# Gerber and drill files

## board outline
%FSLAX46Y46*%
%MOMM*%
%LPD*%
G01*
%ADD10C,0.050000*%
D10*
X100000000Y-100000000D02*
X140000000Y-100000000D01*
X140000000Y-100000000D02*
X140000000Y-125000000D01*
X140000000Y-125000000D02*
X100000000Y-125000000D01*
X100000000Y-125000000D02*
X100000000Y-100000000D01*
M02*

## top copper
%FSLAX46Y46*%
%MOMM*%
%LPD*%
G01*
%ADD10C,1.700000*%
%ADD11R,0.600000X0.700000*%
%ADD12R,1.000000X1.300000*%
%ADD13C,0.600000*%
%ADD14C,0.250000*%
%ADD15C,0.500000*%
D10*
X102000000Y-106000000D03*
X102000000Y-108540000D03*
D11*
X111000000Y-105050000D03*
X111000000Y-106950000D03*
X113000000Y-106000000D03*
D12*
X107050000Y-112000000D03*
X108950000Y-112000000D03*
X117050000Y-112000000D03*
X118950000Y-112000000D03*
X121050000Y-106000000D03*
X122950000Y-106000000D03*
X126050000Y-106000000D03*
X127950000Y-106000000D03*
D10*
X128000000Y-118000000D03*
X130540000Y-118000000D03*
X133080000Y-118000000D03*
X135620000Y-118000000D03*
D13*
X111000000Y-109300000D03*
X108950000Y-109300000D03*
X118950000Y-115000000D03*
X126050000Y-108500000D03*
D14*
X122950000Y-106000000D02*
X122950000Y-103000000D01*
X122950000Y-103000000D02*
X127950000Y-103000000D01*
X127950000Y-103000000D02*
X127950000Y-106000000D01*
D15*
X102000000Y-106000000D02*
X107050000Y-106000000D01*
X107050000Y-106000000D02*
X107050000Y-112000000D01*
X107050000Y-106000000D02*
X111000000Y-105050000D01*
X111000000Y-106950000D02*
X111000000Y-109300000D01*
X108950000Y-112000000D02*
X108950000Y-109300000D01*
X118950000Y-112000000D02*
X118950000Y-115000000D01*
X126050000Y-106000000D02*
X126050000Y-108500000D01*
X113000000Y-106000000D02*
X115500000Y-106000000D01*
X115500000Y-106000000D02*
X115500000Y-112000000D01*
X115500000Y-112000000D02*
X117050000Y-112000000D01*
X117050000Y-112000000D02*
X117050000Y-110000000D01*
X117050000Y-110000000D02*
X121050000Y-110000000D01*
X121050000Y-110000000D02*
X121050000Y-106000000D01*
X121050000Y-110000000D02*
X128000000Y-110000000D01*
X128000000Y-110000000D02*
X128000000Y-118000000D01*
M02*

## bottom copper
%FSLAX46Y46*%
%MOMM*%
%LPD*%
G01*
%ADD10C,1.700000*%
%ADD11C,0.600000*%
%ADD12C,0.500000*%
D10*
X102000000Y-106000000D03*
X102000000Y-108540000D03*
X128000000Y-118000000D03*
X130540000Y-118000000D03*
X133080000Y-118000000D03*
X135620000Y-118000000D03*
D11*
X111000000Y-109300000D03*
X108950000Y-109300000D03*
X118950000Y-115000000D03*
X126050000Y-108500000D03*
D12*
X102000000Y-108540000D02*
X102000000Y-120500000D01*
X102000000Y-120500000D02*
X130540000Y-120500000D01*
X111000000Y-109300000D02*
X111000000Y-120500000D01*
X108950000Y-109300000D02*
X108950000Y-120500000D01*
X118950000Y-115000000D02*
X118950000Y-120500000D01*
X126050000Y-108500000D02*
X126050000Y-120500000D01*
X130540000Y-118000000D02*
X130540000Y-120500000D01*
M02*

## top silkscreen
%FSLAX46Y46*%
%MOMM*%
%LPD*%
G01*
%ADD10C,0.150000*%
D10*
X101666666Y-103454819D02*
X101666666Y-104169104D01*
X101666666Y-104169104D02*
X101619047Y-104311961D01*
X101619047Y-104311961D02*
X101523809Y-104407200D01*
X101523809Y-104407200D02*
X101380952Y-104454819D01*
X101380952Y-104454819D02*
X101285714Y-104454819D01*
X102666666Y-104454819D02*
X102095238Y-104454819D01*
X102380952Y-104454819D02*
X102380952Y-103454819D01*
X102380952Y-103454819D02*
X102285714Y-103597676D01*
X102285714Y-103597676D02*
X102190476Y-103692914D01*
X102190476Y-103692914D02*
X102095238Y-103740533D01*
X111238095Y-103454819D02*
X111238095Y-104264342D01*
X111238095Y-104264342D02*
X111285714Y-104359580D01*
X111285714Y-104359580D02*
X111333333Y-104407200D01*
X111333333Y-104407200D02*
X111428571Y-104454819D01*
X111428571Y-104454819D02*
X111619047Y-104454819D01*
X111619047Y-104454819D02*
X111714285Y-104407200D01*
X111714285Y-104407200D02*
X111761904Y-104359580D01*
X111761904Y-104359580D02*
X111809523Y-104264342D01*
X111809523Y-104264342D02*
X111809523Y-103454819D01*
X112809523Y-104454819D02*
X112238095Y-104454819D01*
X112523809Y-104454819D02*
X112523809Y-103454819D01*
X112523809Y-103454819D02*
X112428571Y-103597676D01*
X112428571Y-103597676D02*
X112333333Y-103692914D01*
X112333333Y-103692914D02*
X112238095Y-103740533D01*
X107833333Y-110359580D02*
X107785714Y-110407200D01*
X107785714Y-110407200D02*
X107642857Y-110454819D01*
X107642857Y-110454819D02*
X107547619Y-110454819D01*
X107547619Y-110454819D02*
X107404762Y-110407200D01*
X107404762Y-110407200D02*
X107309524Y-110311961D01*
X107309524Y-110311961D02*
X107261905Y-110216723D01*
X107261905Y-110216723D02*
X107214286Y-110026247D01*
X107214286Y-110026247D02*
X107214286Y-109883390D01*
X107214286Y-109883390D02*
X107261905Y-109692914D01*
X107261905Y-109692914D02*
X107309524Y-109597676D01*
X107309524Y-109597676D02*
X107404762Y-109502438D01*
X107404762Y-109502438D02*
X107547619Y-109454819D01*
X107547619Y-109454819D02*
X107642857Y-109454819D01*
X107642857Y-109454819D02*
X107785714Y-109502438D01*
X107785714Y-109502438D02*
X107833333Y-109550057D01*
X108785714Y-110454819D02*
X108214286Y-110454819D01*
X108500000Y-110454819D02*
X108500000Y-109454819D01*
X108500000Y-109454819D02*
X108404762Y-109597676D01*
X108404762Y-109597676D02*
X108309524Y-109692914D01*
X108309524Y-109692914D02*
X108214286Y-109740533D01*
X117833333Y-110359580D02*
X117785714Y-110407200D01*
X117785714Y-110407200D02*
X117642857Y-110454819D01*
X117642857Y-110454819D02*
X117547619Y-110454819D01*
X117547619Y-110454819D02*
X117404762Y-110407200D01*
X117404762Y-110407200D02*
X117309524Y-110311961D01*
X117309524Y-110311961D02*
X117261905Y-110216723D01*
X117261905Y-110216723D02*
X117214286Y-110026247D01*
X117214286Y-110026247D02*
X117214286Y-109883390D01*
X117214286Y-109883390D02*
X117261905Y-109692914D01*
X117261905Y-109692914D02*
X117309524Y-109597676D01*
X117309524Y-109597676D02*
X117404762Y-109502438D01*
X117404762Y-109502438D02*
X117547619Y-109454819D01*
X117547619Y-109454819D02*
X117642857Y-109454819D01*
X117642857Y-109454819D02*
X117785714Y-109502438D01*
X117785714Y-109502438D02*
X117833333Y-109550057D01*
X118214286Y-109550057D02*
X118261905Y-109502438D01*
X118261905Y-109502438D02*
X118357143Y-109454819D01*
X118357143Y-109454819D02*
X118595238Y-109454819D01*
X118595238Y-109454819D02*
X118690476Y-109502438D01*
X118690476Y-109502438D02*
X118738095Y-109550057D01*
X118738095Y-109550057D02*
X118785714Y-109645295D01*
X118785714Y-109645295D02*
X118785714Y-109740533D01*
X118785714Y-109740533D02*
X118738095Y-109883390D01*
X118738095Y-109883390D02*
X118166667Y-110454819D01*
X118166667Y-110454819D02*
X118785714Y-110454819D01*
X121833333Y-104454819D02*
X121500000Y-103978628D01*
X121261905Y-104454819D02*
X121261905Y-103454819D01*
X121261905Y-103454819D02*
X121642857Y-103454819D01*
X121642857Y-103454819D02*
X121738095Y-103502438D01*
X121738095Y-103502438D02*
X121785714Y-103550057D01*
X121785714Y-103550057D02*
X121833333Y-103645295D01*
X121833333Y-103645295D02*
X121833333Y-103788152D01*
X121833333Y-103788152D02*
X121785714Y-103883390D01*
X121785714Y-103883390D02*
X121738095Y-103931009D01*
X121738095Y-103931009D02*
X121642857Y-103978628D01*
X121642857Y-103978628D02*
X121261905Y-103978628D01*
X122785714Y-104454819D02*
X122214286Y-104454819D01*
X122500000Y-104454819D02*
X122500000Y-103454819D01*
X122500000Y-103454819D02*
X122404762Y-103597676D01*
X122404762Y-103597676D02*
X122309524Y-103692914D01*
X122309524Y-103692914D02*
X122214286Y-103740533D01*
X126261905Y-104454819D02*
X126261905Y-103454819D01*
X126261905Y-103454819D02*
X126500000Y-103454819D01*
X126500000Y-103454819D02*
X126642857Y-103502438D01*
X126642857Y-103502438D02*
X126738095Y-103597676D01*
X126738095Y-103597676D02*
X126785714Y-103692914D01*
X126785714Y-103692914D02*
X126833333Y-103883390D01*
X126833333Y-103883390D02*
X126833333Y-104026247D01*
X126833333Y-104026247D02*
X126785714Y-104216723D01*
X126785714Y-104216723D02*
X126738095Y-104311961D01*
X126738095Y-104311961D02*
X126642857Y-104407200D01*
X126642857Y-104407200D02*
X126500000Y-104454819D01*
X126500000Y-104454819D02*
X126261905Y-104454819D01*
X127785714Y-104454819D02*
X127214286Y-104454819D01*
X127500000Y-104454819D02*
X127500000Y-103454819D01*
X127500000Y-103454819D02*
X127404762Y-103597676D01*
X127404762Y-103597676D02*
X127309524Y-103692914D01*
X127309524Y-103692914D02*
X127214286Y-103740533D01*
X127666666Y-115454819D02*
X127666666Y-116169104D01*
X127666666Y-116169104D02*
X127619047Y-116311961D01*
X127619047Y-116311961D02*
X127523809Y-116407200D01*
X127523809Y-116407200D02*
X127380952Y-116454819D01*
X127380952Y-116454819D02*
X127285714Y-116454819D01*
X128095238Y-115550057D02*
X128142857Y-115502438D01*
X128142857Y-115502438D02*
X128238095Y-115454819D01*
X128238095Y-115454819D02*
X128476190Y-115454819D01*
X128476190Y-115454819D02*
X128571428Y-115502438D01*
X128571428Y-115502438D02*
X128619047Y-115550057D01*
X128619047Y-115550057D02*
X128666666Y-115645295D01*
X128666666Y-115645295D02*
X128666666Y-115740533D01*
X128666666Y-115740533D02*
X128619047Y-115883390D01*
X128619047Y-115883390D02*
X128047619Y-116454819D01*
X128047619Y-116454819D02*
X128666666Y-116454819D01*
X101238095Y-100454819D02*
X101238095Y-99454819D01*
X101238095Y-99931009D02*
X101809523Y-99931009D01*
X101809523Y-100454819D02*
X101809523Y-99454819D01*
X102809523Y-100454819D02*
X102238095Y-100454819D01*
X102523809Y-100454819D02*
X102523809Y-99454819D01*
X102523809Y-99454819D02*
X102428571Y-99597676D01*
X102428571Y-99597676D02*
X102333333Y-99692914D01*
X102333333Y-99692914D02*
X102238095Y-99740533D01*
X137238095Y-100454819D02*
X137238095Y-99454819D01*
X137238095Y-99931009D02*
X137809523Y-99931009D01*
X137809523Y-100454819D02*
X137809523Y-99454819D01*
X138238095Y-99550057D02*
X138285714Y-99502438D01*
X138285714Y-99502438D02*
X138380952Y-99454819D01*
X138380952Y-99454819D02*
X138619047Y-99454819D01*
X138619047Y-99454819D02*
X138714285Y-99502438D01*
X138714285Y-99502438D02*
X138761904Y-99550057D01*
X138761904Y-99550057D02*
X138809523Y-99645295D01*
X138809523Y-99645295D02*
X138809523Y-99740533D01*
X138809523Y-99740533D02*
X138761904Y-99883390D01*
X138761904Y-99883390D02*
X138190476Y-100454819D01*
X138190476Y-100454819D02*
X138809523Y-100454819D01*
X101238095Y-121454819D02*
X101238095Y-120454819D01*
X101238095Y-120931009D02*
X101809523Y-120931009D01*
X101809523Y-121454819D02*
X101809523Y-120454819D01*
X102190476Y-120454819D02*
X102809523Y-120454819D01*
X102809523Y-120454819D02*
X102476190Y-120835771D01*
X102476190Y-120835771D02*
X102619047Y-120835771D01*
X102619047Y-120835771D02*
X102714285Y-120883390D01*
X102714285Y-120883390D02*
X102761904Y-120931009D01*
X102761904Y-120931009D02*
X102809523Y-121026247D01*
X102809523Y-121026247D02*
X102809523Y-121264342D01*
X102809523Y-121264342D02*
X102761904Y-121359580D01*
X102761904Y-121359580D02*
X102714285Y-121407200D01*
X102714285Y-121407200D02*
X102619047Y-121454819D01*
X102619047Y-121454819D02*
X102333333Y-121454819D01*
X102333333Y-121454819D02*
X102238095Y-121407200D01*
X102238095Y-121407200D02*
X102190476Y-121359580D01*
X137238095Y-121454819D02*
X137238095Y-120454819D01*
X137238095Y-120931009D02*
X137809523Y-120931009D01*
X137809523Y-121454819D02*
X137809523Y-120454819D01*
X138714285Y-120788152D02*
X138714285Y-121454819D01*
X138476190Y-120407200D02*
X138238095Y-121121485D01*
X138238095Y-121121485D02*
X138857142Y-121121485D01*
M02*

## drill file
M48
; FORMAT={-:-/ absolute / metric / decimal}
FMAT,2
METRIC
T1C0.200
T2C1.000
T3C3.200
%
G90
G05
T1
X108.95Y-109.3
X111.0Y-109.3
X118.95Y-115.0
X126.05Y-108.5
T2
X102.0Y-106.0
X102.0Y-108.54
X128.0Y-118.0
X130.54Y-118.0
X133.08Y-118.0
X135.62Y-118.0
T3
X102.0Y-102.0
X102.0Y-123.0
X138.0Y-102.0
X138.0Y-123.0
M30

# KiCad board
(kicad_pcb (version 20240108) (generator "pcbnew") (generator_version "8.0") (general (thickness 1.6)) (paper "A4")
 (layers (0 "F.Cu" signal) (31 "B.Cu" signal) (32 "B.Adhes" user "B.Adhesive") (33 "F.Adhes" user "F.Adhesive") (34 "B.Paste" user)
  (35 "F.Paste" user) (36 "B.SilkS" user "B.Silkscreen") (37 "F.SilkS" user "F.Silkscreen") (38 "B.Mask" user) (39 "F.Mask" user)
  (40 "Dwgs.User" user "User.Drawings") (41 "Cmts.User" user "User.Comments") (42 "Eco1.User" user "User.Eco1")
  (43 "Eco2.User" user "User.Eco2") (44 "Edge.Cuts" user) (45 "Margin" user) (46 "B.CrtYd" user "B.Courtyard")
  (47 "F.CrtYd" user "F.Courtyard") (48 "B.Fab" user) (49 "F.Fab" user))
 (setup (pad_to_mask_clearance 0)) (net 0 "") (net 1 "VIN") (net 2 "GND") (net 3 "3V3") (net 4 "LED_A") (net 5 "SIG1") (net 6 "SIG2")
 (gr_line (start 100 100) (end 140 100) (stroke (width 0.05) (type default)) (layer "Edge.Cuts"))
 (gr_line (start 140 100) (end 140 125) (stroke (width 0.05) (type default)) (layer "Edge.Cuts"))
 (gr_line (start 140 125) (end 100 125) (stroke (width 0.05) (type default)) (layer "Edge.Cuts"))
 (gr_line (start 100 125) (end 100 100) (stroke (width 0.05) (type default)) (layer "Edge.Cuts"))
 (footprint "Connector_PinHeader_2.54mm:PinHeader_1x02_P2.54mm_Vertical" (layer "F.Cu") (at 102 106)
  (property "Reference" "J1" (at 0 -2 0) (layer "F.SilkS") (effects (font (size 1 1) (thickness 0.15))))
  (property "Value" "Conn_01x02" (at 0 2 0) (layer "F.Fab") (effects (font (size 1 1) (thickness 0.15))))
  (pad "1" thru_hole circle (at 0 0) (size 1.7 1.7) (drill 1) (layers "*.Cu" "*.Mask") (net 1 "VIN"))
  (pad "2" thru_hole circle (at 0 2.54) (size 1.7 1.7) (drill 1) (layers "*.Cu" "*.Mask") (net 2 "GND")))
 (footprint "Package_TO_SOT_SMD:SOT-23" (layer "F.Cu") (at 112 106)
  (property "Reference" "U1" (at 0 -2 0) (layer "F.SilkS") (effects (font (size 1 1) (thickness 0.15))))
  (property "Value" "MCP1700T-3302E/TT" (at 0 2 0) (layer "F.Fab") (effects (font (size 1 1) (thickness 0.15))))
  (pad "1" smd rect (at -1 -0.95) (size 0.6 0.7) (layers "F.Cu" "F.Paste" "F.Mask") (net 1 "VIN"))
  (pad "2" smd rect (at -1 0.95) (size 0.6 0.7) (layers "F.Cu" "F.Paste" "F.Mask") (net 2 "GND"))
  (pad "3" smd rect (at 1 0) (size 0.6 0.7) (layers "F.Cu" "F.Paste" "F.Mask") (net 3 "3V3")))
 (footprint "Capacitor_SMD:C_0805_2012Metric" (layer "F.Cu") (at 108 112)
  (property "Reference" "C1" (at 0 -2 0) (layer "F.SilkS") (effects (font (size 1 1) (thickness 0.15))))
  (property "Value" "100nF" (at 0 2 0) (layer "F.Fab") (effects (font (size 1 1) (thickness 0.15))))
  (pad "1" smd rect (at -0.95 0) (size 1 1.3) (layers "F.Cu" "F.Paste" "F.Mask") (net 1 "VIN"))
  (pad "2" smd rect (at 0.95 0) (size 1 1.3) (layers "F.Cu" "F.Paste" "F.Mask") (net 2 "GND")))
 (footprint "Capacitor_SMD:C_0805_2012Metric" (layer "F.Cu") (at 118 112)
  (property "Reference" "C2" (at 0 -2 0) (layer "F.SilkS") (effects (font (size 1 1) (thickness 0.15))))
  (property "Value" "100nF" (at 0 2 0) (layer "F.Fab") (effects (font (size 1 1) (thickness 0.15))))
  (pad "1" smd rect (at -0.95 0) (size 1 1.3) (layers "F.Cu" "F.Paste" "F.Mask") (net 3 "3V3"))
  (pad "2" smd rect (at 0.95 0) (size 1 1.3) (layers "F.Cu" "F.Paste" "F.Mask") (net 2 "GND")))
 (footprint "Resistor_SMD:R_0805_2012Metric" (layer "F.Cu") (at 122 106)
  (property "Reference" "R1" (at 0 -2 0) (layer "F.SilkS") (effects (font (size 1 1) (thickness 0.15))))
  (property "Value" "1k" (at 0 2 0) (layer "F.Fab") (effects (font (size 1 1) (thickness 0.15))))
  (pad "1" smd rect (at -0.95 0) (size 1 1.3) (layers "F.Cu" "F.Paste" "F.Mask") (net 3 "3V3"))
  (pad "2" smd rect (at 0.95 0) (size 1 1.3) (layers "F.Cu" "F.Paste" "F.Mask") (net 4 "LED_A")))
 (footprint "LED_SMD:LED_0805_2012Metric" (layer "F.Cu") (at 127 106)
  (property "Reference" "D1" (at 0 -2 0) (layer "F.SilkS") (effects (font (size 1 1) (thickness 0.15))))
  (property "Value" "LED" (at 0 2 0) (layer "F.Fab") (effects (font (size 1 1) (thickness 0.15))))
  (pad "1" smd rect (at -0.95 0) (size 1 1.3) (layers "F.Cu" "F.Paste" "F.Mask") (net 2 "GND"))
  (pad "2" smd rect (at 0.95 0) (size 1 1.3) (layers "F.Cu" "F.Paste" "F.Mask") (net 4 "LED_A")))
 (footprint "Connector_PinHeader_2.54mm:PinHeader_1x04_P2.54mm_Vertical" (layer "F.Cu") (at 128 118)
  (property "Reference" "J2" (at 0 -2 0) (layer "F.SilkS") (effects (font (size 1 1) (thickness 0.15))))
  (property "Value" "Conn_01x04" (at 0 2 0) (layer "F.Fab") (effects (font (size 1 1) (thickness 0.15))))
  (pad "1" thru_hole circle (at 0 0) (size 1.7 1.7) (drill 1) (layers "*.Cu" "*.Mask") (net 3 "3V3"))
  (pad "2" thru_hole circle (at 2.54 0) (size 1.7 1.7) (drill 1) (layers "*.Cu" "*.Mask") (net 2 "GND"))
  (pad "3" thru_hole circle (at 5.08 0) (size 1.7 1.7) (drill 1) (layers "*.Cu" "*.Mask") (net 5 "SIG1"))
  (pad "4" thru_hole circle (at 7.62 0) (size 1.7 1.7) (drill 1) (layers "*.Cu" "*.Mask") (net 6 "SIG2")))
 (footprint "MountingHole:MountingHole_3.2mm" (layer "F.Cu") (at 102 102)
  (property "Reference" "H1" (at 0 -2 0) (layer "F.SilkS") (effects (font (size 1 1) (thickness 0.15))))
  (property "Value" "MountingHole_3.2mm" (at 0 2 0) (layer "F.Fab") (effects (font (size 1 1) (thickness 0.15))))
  (pad "1" np_thru_hole circle (at 0 0) (size 3.2 3.2) (drill 3.2) (layers "*.Cu" "*.Mask")))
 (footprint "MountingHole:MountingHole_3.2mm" (layer "F.Cu") (at 138 102)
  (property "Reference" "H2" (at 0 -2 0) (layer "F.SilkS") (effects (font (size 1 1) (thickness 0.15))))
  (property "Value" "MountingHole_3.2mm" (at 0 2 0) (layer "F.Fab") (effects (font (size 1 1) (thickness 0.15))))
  (pad "1" np_thru_hole circle (at 0 0) (size 3.2 3.2) (drill 3.2) (layers "*.Cu" "*.Mask")))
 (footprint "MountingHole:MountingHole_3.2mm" (layer "F.Cu") (at 102 123)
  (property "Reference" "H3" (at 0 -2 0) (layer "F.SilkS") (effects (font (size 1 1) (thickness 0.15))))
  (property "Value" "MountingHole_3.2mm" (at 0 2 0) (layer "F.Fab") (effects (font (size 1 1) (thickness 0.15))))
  (pad "1" np_thru_hole circle (at 0 0) (size 3.2 3.2) (drill 3.2) (layers "*.Cu" "*.Mask")))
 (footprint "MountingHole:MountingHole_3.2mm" (layer "F.Cu") (at 138 123)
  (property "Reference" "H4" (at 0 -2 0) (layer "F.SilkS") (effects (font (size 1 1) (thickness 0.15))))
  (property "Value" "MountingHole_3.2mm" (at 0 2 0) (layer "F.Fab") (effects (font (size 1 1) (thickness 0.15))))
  (pad "1" np_thru_hole circle (at 0 0) (size 3.2 3.2) (drill 3.2) (layers "*.Cu" "*.Mask")))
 (segment (start 122.95 106) (end 122.95 103) (width 0.25) (layer "F.Cu") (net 4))
 (segment (start 122.95 103) (end 127.95 103) (width 0.25) (layer "F.Cu") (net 4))
 (segment (start 127.95 103) (end 127.95 106) (width 0.25) (layer "F.Cu") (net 4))
 (segment (start 102 106) (end 107.05 106) (width 0.5) (layer "F.Cu") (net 1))
 (segment (start 107.05 106) (end 107.05 112) (width 0.5) (layer "F.Cu") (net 1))
 (segment (start 107.05 106) (end 111 105.05) (width 0.5) (layer "F.Cu") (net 1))
 (segment (start 111 106.95) (end 111 109.3) (width 0.5) (layer "F.Cu") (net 2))
 (segment (start 108.95 112) (end 108.95 109.3) (width 0.5) (layer "F.Cu") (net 2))
 (segment (start 118.95 112) (end 118.95 115) (width 0.5) (layer "F.Cu") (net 2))
 (segment (start 126.05 106) (end 126.05 108.5) (width 0.5) (layer "F.Cu") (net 2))
 (segment (start 113 106) (end 115.5 106) (width 0.5) (layer "F.Cu") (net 3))
 (segment (start 115.5 106) (end 115.5 112) (width 0.5) (layer "F.Cu") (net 3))
 (segment (start 115.5 112) (end 117.05 112) (width 0.5) (layer "F.Cu") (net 3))
 (segment (start 117.05 112) (end 117.05 110) (width 0.5) (layer "F.Cu") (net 3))
 (segment (start 117.05 110) (end 121.05 110) (width 0.5) (layer "F.Cu") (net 3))
 (segment (start 121.05 110) (end 121.05 106) (width 0.5) (layer "F.Cu") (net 3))
 (segment (start 121.05 110) (end 128 110) (width 0.5) (layer "F.Cu") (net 3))
 (segment (start 128 110) (end 128 118) (width 0.5) (layer "F.Cu") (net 3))
 (segment (start 102 108.54) (end 102 120.5) (width 0.5) (layer "B.Cu") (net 2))
 (segment (start 102 120.5) (end 130.54 120.5) (width 0.5) (layer "B.Cu") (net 2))
 (segment (start 111 109.3) (end 111 120.5) (width 0.5) (layer "B.Cu") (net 2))
 (segment (start 108.95 109.3) (end 108.95 120.5) (width 0.5) (layer "B.Cu") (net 2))
 (segment (start 118.95 115) (end 118.95 120.5) (width 0.5) (layer "B.Cu") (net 2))
 (segment (start 126.05 108.5) (end 126.05 120.5) (width 0.5) (layer "B.Cu") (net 2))
 (segment (start 130.54 118) (end 130.54 120.5) (width 0.5) (layer "B.Cu") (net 2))
 (via (at 111 109.3) (size 0.6) (drill 0.2) (layers "F.Cu" "B.Cu") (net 2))
 (via (at 108.95 109.3) (size 0.6) (drill 0.2) (layers "F.Cu" "B.Cu") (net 2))
 (via (at 118.95 115) (size 0.6) (drill 0.2) (layers "F.Cu" "B.Cu") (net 2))
 (via (at 126.05 108.5) (size 0.6) (drill 0.2) (layers "F.Cu" "B.Cu") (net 2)))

